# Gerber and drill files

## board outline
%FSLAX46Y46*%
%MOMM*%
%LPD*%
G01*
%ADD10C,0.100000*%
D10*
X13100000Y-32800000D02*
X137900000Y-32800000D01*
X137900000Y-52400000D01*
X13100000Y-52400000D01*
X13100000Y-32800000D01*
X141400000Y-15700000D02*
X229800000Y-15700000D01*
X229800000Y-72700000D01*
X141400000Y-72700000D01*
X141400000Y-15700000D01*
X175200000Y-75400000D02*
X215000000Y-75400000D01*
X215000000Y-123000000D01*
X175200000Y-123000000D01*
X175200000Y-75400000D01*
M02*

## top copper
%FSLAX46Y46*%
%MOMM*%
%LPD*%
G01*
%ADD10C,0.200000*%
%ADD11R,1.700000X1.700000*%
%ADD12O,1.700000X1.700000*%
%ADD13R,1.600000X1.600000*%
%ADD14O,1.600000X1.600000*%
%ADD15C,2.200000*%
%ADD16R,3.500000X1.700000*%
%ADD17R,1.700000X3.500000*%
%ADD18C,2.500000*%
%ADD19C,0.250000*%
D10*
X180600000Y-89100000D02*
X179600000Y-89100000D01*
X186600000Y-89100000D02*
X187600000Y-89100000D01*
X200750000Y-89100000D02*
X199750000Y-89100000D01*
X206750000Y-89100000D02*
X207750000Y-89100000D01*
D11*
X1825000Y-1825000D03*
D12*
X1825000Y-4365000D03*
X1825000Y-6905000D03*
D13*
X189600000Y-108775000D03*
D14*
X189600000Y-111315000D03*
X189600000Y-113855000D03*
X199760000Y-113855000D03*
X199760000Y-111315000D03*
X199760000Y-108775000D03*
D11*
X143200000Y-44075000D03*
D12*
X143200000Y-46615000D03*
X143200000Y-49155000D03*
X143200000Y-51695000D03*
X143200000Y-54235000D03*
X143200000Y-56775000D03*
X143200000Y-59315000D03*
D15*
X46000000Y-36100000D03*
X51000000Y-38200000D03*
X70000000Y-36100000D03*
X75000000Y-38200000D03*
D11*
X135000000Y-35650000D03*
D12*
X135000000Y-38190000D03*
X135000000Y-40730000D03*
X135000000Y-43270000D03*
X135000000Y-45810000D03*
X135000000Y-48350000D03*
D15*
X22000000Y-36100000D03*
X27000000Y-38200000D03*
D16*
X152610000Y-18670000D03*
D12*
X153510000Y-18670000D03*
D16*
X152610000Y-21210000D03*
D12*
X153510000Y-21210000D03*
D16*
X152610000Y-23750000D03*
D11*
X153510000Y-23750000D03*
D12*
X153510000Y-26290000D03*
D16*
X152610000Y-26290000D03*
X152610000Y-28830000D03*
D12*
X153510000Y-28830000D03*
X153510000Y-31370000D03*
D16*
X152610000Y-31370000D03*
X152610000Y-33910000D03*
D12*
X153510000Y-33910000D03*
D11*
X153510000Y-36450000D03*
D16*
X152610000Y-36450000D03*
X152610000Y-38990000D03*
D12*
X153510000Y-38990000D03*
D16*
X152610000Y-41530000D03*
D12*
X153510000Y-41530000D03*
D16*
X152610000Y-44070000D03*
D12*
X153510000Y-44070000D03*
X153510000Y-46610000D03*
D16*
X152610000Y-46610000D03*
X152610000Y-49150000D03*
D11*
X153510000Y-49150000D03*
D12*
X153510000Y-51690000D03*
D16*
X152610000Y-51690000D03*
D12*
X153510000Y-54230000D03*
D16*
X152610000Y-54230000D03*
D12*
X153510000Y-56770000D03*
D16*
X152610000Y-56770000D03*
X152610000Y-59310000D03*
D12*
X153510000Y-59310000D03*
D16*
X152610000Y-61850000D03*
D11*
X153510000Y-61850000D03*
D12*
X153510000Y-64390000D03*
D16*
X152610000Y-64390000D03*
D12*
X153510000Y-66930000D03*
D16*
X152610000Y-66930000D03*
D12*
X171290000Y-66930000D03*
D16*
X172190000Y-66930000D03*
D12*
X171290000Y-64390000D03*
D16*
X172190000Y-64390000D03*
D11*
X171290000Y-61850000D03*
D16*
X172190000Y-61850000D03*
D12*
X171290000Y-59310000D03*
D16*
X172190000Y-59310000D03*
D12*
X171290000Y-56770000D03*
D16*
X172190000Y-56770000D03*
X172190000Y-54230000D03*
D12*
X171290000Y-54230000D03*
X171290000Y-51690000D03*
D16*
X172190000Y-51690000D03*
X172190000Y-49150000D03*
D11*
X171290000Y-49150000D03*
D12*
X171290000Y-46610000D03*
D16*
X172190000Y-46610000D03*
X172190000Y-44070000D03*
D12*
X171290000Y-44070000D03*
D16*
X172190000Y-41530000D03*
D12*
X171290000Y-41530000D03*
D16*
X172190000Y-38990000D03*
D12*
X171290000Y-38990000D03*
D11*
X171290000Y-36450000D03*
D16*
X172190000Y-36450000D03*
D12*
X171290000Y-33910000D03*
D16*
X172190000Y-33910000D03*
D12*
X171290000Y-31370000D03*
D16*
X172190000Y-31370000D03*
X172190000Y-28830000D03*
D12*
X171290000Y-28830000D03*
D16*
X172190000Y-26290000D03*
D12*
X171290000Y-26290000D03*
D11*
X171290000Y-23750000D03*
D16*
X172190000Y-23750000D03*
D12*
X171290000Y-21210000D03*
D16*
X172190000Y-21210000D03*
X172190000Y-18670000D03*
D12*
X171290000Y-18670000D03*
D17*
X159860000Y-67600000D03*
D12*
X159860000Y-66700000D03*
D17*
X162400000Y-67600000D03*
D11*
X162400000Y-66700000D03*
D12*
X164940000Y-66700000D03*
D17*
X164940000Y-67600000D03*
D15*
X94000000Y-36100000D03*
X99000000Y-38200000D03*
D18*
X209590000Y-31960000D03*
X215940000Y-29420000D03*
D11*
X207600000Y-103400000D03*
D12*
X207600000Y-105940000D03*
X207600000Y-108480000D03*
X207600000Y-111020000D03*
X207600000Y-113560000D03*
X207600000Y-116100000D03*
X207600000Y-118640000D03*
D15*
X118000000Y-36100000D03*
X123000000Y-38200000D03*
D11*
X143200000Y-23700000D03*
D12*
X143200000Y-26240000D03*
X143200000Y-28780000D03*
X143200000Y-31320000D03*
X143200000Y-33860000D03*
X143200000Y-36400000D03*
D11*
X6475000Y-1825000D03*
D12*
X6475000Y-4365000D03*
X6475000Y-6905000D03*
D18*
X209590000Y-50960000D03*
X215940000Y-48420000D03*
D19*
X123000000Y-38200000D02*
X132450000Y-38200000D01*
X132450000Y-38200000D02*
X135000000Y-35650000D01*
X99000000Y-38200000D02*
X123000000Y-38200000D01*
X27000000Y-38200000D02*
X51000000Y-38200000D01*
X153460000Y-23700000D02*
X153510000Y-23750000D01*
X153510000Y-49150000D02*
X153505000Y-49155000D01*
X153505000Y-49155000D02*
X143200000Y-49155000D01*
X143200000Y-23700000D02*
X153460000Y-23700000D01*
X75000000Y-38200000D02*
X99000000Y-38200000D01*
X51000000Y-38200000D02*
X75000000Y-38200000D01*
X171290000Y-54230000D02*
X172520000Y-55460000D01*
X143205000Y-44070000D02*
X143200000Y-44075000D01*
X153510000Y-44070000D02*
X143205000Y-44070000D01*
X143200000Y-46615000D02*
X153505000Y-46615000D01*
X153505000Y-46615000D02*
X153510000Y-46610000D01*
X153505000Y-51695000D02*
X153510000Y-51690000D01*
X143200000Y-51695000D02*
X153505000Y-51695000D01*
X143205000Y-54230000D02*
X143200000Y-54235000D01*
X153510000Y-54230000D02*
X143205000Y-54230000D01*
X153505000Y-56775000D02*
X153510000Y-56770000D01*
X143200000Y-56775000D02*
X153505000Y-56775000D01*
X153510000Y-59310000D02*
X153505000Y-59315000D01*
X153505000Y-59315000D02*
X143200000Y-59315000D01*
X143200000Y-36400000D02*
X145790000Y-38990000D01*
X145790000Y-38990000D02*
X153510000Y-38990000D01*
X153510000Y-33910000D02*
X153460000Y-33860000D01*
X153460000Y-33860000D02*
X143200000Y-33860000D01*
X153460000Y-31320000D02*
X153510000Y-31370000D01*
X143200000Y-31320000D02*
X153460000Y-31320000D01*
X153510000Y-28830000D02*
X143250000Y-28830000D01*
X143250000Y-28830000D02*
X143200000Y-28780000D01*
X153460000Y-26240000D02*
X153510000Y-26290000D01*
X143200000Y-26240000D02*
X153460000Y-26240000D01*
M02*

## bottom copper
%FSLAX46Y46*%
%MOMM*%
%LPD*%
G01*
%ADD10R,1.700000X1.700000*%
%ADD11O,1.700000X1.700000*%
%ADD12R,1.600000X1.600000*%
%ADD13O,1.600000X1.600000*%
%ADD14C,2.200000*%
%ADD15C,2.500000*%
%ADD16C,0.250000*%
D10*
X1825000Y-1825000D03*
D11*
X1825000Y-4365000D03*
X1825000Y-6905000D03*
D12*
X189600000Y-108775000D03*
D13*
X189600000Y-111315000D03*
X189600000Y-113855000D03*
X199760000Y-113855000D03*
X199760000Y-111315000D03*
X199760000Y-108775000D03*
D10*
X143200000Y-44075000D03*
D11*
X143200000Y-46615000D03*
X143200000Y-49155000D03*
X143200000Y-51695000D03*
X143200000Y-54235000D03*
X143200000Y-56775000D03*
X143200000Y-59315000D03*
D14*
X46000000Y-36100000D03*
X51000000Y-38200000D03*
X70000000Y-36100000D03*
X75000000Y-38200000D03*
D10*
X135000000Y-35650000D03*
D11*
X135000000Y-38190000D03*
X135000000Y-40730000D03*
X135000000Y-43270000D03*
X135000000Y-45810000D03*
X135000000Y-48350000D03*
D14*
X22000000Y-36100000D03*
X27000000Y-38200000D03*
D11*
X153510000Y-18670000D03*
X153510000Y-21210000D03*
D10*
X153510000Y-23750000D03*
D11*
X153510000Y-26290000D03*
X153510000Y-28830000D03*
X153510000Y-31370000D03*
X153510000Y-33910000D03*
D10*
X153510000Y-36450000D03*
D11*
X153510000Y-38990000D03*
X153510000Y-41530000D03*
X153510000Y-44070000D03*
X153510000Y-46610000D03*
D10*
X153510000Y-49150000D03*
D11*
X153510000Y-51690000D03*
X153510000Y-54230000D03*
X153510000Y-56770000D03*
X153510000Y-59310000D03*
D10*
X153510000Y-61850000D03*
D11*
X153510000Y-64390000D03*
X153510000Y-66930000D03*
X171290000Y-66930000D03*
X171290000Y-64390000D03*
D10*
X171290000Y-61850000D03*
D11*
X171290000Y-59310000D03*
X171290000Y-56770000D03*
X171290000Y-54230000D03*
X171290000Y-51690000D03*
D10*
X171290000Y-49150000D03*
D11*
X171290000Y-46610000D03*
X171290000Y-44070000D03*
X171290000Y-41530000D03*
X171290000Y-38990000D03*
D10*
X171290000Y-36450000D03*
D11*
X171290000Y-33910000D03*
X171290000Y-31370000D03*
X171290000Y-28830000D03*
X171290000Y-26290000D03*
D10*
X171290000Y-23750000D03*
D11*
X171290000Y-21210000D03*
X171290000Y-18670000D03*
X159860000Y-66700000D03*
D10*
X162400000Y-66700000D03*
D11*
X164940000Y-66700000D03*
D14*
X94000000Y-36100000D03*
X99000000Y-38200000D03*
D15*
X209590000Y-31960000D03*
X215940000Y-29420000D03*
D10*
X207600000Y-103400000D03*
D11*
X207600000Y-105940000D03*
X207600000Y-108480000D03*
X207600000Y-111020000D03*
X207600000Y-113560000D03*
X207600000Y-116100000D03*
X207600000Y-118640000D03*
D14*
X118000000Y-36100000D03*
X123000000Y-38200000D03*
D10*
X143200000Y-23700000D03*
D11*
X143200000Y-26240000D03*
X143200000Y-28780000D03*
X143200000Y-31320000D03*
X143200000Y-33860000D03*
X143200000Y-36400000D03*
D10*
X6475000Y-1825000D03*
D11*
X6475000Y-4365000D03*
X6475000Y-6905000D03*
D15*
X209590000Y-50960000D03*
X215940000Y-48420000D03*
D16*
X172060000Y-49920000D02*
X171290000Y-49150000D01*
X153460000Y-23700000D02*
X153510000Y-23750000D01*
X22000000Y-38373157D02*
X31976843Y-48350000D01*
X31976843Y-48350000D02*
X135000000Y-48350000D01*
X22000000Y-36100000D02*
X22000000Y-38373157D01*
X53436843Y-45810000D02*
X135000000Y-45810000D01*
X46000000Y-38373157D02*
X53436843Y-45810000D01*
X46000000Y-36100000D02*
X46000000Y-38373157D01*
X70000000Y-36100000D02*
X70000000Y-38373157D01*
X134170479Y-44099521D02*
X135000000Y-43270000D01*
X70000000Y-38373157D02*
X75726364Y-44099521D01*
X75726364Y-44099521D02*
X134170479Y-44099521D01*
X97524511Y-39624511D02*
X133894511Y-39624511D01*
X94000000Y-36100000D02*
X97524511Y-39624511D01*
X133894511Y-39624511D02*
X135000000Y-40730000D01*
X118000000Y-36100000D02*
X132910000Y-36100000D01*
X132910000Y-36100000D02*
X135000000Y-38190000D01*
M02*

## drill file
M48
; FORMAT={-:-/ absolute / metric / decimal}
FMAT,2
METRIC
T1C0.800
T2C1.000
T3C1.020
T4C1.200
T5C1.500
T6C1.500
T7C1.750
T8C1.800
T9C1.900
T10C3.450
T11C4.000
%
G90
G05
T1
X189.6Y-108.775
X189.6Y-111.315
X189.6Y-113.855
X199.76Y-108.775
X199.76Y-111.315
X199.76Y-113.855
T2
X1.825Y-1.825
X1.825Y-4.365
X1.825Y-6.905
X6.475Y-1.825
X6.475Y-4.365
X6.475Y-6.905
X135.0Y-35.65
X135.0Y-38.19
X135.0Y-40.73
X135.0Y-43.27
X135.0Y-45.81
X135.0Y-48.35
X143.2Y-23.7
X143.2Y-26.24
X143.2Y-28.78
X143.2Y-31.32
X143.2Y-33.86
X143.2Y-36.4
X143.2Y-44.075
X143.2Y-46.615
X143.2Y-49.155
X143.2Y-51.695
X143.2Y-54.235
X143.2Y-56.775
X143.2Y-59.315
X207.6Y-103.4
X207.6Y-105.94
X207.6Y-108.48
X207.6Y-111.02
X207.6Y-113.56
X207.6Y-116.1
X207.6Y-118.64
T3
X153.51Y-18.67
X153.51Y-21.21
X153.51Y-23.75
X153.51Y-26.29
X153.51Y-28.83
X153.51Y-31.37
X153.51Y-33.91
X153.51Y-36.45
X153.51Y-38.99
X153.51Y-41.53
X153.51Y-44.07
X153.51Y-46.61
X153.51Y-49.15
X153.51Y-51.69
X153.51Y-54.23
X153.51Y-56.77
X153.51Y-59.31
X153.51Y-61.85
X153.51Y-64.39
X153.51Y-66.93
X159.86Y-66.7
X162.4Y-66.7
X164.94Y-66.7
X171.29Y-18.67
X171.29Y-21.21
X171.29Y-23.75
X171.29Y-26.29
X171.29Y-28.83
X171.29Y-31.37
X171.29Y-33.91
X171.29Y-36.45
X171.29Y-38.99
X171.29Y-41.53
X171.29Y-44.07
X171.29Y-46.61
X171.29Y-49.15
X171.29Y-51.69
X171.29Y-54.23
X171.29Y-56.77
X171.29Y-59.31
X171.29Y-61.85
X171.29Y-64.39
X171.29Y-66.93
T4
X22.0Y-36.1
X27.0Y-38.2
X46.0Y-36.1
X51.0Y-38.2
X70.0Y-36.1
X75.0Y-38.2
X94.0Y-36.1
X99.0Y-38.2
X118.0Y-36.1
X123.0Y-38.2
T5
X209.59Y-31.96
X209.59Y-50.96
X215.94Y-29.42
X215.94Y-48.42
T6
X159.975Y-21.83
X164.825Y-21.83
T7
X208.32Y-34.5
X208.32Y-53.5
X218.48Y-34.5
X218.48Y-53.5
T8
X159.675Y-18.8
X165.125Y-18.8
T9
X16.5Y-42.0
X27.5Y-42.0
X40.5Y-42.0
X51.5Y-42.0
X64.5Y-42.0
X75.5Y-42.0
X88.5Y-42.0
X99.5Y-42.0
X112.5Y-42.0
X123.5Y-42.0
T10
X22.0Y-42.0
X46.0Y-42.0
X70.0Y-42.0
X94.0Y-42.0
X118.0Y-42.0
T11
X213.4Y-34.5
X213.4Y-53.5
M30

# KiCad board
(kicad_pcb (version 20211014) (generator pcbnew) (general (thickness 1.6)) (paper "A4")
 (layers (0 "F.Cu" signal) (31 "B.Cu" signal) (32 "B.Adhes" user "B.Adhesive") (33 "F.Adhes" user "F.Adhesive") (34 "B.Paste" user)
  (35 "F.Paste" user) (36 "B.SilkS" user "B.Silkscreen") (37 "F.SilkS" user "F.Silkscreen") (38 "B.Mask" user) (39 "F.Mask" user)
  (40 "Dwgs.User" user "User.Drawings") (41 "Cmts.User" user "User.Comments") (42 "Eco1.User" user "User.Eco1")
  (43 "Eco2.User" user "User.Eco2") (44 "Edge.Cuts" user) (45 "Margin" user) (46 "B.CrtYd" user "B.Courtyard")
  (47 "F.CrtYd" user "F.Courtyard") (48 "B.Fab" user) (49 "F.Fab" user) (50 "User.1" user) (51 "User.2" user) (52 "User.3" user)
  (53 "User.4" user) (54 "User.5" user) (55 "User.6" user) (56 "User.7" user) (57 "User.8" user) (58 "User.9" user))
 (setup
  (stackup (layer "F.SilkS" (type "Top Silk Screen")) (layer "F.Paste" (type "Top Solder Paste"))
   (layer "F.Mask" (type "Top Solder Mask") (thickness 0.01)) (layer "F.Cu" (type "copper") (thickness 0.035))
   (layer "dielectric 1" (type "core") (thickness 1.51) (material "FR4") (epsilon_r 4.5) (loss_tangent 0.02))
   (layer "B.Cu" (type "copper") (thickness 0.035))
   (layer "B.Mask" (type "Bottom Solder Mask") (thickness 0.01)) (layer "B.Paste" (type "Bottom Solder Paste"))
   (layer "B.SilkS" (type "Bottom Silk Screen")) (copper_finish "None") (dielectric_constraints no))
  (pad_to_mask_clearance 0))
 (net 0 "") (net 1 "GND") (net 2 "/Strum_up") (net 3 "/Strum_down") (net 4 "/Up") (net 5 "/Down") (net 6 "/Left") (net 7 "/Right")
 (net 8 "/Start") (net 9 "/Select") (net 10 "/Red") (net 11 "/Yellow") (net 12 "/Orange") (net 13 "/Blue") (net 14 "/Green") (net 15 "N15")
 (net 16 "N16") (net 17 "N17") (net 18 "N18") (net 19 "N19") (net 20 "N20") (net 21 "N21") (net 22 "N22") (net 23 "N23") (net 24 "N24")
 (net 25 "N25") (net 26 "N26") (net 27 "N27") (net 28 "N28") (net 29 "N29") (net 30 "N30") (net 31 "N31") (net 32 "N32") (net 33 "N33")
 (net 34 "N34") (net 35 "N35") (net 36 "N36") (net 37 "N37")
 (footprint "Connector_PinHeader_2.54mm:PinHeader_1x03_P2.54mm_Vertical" (layer "F.Cu") (at 1.825 1.825)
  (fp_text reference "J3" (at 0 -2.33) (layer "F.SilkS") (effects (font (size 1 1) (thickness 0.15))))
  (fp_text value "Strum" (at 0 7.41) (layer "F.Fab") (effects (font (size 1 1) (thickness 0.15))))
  (pad "1" thru_hole rect (at 0 0) (size 1.7 1.7) (drill 1) (layers *.Cu *.Mask) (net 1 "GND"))
  (pad "2" thru_hole oval (at 0 2.54) (size 1.7 1.7) (drill 1) (layers *.Cu *.Mask) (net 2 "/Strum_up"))
  (pad "3" thru_hole oval (at 0 5.08) (size 1.7 1.7) (drill 1) (layers *.Cu *.Mask) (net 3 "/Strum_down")))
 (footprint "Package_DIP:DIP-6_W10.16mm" (layer "F.Cu") (at 189.6 108.775)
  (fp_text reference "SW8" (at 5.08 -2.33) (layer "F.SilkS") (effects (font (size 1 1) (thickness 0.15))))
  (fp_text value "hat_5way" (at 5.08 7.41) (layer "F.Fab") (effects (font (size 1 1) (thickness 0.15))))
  (pad "1" thru_hole rect (at 0 0) (size 1.6 1.6) (drill 0.8) (layers *.Cu *.Mask) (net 1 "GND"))
  (pad "2" thru_hole oval (at 0 2.54) (size 1.6 1.6) (drill 0.8) (layers *.Cu *.Mask) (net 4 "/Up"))
  (pad "3" thru_hole oval (at 0 5.08) (size 1.6 1.6) (drill 0.8) (layers *.Cu *.Mask) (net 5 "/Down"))
  (pad "4" thru_hole oval (at 10.16 5.08) (size 1.6 1.6) (drill 0.8) (layers *.Cu *.Mask) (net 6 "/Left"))
  (pad "5" thru_hole oval (at 10.16 2.54) (size 1.6 1.6) (drill 0.8) (layers *.Cu *.Mask) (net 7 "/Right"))
  (pad "6" thru_hole oval (at 10.16 0) (size 1.6 1.6) (drill 0.8) (layers *.Cu *.Mask)))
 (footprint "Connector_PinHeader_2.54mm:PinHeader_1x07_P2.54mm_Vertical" (layer "F.Cu") (at 143.2 44.075)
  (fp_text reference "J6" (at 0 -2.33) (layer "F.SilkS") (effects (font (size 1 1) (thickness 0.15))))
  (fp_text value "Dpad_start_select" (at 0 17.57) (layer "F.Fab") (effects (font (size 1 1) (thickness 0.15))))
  (pad "1" thru_hole rect (at 0 0) (size 1.7 1.7) (drill 1) (layers *.Cu *.Mask) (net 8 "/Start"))
  (pad "2" thru_hole oval (at 0 2.54) (size 1.7 1.7) (drill 1) (layers *.Cu *.Mask) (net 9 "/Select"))
  (pad "3" thru_hole oval (at 0 5.08) (size 1.7 1.7) (drill 1) (layers *.Cu *.Mask) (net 1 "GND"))
  (pad "4" thru_hole oval (at 0 7.62) (size 1.7 1.7) (drill 1) (layers *.Cu *.Mask) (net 4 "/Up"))
  (pad "5" thru_hole oval (at 0 10.16) (size 1.7 1.7) (drill 1) (layers *.Cu *.Mask) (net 5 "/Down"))
  (pad "6" thru_hole oval (at 0 12.7) (size 1.7 1.7) (drill 1) (layers *.Cu *.Mask) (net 6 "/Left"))
  (pad "7" thru_hole oval (at 0 15.24) (size 1.7 1.7) (drill 1) (layers *.Cu *.Mask) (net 7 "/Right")))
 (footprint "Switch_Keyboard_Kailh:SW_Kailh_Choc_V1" (layer "F.Cu") (at 46 42)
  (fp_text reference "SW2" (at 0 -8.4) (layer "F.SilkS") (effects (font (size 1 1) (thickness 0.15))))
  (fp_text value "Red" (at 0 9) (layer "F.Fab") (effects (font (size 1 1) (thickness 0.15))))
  (pad "" np_thru_hole circle locked (at 5.5 0) (size 1.9 1.9) (drill 1.9) (layers *.Cu *.Mask))
  (pad "" np_thru_hole circle locked (at -5.5 0) (size 1.9 1.9) (drill 1.9) (layers *.Cu *.Mask))
  (pad "" smd circle locked (at 0 -5.9) (size 1.25 1.25) (layers "F.Mask"))
  (pad "" np_thru_hole circle locked (at 0 0) (size 3.45 3.45) (drill 3.45) (layers *.Cu *.Mask))
  (pad "" smd circle locked (at 5 -3.8) (size 1.25 1.25) (layers "F.Mask"))
  (pad "1" thru_hole circle locked (at 0 -5.9) (size 2.2 2.2) (drill 1.2) (layers *.Cu "B.Mask") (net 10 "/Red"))
  (pad "2" thru_hole circle locked (at 5 -3.8) (size 2.2 2.2) (drill 1.2) (layers *.Cu "B.Mask") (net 1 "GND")))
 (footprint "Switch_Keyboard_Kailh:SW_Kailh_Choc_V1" (layer "F.Cu") (at 70 42)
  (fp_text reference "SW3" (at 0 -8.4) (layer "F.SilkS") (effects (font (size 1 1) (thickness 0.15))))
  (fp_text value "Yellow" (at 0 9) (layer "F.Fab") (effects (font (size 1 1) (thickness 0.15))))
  (pad "" np_thru_hole circle locked (at -5.5 0) (size 1.9 1.9) (drill 1.9) (layers *.Cu *.Mask))
  (pad "" np_thru_hole circle locked (at 0 0) (size 3.45 3.45) (drill 3.45) (layers *.Cu *.Mask))
  (pad "" smd circle locked (at 0 -5.9) (size 1.25 1.25) (layers "F.Mask"))
  (pad "" smd circle locked (at 5 -3.8) (size 1.25 1.25) (layers "F.Mask"))
  (pad "" np_thru_hole circle locked (at 5.5 0) (size 1.9 1.9) (drill 1.9) (layers *.Cu *.Mask))
  (pad "1" thru_hole circle locked (at 0 -5.9) (size 2.2 2.2) (drill 1.2) (layers *.Cu "B.Mask") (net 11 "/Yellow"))
  (pad "2" thru_hole circle locked (at 5 -3.8) (size 2.2 2.2) (drill 1.2) (layers *.Cu "B.Mask") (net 1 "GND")))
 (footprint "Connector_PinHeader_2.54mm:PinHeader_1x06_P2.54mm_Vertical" (layer "F.Cu") (at 135 35.65)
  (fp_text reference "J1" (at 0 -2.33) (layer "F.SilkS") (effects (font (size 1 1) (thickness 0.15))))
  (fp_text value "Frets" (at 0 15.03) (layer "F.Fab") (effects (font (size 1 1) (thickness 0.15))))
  (pad "1" thru_hole rect (at 0 0) (size 1.7 1.7) (drill 1) (layers *.Cu *.Mask) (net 1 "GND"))
  (pad "2" thru_hole oval (at 0 2.54) (size 1.7 1.7) (drill 1) (layers *.Cu *.Mask) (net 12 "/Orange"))
  (pad "3" thru_hole oval (at 0 5.08) (size 1.7 1.7) (drill 1) (layers *.Cu *.Mask) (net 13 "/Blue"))
  (pad "4" thru_hole oval (at 0 7.62) (size 1.7 1.7) (drill 1) (layers *.Cu *.Mask) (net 11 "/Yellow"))
  (pad "5" thru_hole oval (at 0 10.16) (size 1.7 1.7) (drill 1) (layers *.Cu *.Mask) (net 10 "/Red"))
  (pad "6" thru_hole oval (at 0 12.7) (size 1.7 1.7) (drill 1) (layers *.Cu *.Mask) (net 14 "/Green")))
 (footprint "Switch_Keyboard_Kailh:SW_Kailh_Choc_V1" (layer "F.Cu") (at 22 42)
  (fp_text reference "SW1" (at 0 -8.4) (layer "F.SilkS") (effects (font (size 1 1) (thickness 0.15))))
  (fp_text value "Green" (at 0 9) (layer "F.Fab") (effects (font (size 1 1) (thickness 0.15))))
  (pad "" smd circle locked (at 0 -5.9) (size 1.25 1.25) (layers "F.Mask"))
  (pad "" smd circle locked (at 5 -3.8) (size 1.25 1.25) (layers "F.Mask"))
  (pad "" np_thru_hole circle locked (at 0 0) (size 3.45 3.45) (drill 3.45) (layers *.Cu *.Mask))
  (pad "" np_thru_hole circle locked (at 5.5 0) (size 1.9 1.9) (drill 1.9) (layers *.Cu *.Mask))
  (pad "" np_thru_hole circle locked (at -5.5 0) (size 1.9 1.9) (drill 1.9) (layers *.Cu *.Mask))
  (pad "1" thru_hole circle locked (at 0 -5.9) (size 2.2 2.2) (drill 1.2) (layers *.Cu "B.Mask") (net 14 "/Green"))
  (pad "2" thru_hole circle locked (at 5 -3.8) (size 2.2 2.2) (drill 1.2) (layers *.Cu "B.Mask") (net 1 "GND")))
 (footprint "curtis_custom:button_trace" (layer "F.Cu") (at 183.6 89.1)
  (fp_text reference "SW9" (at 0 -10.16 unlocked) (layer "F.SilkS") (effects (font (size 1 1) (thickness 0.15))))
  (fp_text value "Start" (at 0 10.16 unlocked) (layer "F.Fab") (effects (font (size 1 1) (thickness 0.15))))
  (fp_line (start -3 0) (end -4 0) (layer "F.Cu") (width 0.2)) (fp_line (start 3 0) (end 4 0) (layer "F.Cu") (width 0.2)))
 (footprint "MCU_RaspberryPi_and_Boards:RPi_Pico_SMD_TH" (layer "F.Cu") (at 162.4 42.8)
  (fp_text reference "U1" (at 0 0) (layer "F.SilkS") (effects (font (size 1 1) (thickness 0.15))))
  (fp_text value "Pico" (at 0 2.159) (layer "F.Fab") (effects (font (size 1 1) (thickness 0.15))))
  (pad "" np_thru_hole oval (at -2.725 -24) (size 1.8 1.8) (drill 1.8) (layers *.Cu *.Mask))
  (pad "" np_thru_hole oval (at 2.425 -20.97) (size 1.5 1.5) (drill 1.5) (layers *.Cu *.Mask))
  (pad "" np_thru_hole oval (at -2.425 -20.97) (size 1.5 1.5) (drill 1.5) (layers *.Cu *.Mask))
  (pad "" np_thru_hole oval (at 2.725 -24) (size 1.8 1.8) (drill 1.8) (layers *.Cu *.Mask))
  (pad "1" smd rect (at -8.89 -24.13) (size 3.5 1.7) (drill (offset -0.9 0)) (layers "F.Cu" "F.Mask") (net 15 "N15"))
  (pad "1" thru_hole oval (at -8.89 -24.13) (size 1.7 1.7) (drill 1.02) (layers *.Cu *.Mask) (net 15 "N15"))
  (pad "2" smd rect (at -8.89 -21.59) (size 3.5 1.7) (drill (offset -0.9 0)) (layers "F.Cu" "F.Mask") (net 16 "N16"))
  (pad "2" thru_hole oval (at -8.89 -21.59) (size 1.7 1.7) (drill 1.02) (layers *.Cu *.Mask) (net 16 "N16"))
  (pad "3" smd rect (at -8.89 -19.05) (size 3.5 1.7) (drill (offset -0.9 0)) (layers "F.Cu" "F.Mask") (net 1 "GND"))
  (pad "3" thru_hole rect (at -8.89 -19.05) (size 1.7 1.7) (drill 1.02) (layers *.Cu *.Mask) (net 1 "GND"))
  (pad "4" thru_hole oval (at -8.89 -16.51) (size 1.7 1.7) (drill 1.02) (layers *.Cu *.Mask) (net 12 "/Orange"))
  (pad "4" smd rect (at -8.89 -16.51) (size 3.5 1.7) (drill (offset -0.9 0)) (layers "F.Cu" "F.Mask") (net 12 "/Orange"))
  (pad "5" smd rect (at -8.89 -13.97) (size 3.5 1.7) (drill (offset -0.9 0)) (layers "F.Cu" "F.Mask") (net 13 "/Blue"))
  (pad "5" thru_hole oval (at -8.89 -13.97) (size 1.7 1.7) (drill 1.02) (layers *.Cu *.Mask) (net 13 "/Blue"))
  (pad "6" thru_hole oval (at -8.89 -11.43) (size 1.7 1.7) (drill 1.02) (layers *.Cu *.Mask) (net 11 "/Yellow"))
  (pad "6" smd rect (at -8.89 -11.43) (size 3.5 1.7) (drill (offset -0.9 0)) (layers "F.Cu" "F.Mask") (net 11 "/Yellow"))
  (pad "7" smd rect (at -8.89 -8.89) (size 3.5 1.7) (drill (offset -0.9 0)) (layers "F.Cu" "F.Mask") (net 10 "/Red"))
  (pad "7" thru_hole oval (at -8.89 -8.89) (size 1.7 1.7) (drill 1.02) (layers *.Cu *.Mask) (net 10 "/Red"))
  (pad "8" thru_hole rect (at -8.89 -6.35) (size 1.7 1.7) (drill 1.02) (layers *.Cu *.Mask) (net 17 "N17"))
  (pad "8" smd rect (at -8.89 -6.35) (size 3.5 1.7) (drill (offset -0.9 0)) (layers "F.Cu" "F.Mask") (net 17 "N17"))
  (pad "9" smd rect (at -8.89 -3.81) (size 3.5 1.7) (drill (offset -0.9 0)) (layers "F.Cu" "F.Mask") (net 14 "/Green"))
  (pad "9" thru_hole oval (at -8.89 -3.81) (size 1.7 1.7) (drill 1.02) (layers *.Cu *.Mask) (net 14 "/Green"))
  (pad "10" smd rect (at -8.89 -1.27) (size 3.5 1.7) (drill (offset -0.9 0)) (layers "F.Cu" "F.Mask") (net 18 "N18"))
  (pad "10" thru_hole oval (at -8.89 -1.27) (size 1.7 1.7) (drill 1.02) (layers *.Cu *.Mask) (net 18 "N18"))
  (pad "11" smd rect (at -8.89 1.27) (size 3.5 1.7) (drill (offset -0.9 0)) (layers "F.Cu" "F.Mask") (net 8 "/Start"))
  (pad "11" thru_hole oval (at -8.89 1.27) (size 1.7 1.7) (drill 1.02) (layers *.Cu *.Mask) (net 8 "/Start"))
  (pad "12" thru_hole oval (at -8.89 3.81) (size 1.7 1.7) (drill 1.02) (layers *.Cu *.Mask) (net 9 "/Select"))
  (pad "12" smd rect (at -8.89 3.81) (size 3.5 1.7) (drill (offset -0.9 0)) (layers "F.Cu" "F.Mask") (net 9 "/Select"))
  (pad "13" smd rect (at -8.89 6.35) (size 3.5 1.7) (drill (offset -0.9 0)) (layers "F.Cu" "F.Mask") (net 1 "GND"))
  (pad "13" thru_hole rect (at -8.89 6.35) (size 1.7 1.7) (drill 1.02) (layers *.Cu *.Mask) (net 1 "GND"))
  (pad "14" thru_hole oval (at -8.89 8.89) (size 1.7 1.7) (drill 1.02) (layers *.Cu *.Mask) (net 4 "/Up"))
  (pad "14" smd rect (at -8.89 8.89) (size 3.5 1.7) (drill (offset -0.9 0)) (layers "F.Cu" "F.Mask") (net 4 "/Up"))
  (pad "15" thru_hole oval (at -8.89 11.43) (size 1.7 1.7) (drill 1.02) (layers *.Cu *.Mask) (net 5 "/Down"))
  (pad "15" smd rect (at -8.89 11.43) (size 3.5 1.7) (drill (offset -0.9 0)) (layers "F.Cu" "F.Mask") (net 5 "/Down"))
  (pad "16" thru_hole oval (at -8.89 13.97) (size 1.7 1.7) (drill 1.02) (layers *.Cu *.Mask) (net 6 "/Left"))
  (pad "16" smd rect (at -8.89 13.97) (size 3.5 1.7) (drill (offset -0.9 0)) (layers "F.Cu" "F.Mask") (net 6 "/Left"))
  (pad "17" smd rect (at -8.89 16.51) (size 3.5 1.7) (drill (offset -0.9 0)) (layers "F.Cu" "F.Mask") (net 7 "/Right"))
  (pad "17" thru_hole oval (at -8.89 16.51) (size 1.7 1.7) (drill 1.02) (layers *.Cu *.Mask) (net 7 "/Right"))
  (pad "18" smd rect (at -8.89 19.05) (size 3.5 1.7) (drill (offset -0.9 0)) (layers "F.Cu" "F.Mask") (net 1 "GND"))
  (pad "18" thru_hole rect (at -8.89 19.05) (size 1.7 1.7) (drill 1.02) (layers *.Cu *.Mask) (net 1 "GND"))
  (pad "19" thru_hole oval (at -8.89 21.59) (size 1.7 1.7) (drill 1.02) (layers *.Cu *.Mask) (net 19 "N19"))
  (pad "19" smd rect (at -8.89 21.59) (size 3.5 1.7) (drill (offset -0.9 0)) (layers "F.Cu" "F.Mask") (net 19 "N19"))
  (pad "20" thru_hole oval (at -8.89 24.13) (size 1.7 1.7) (drill 1.02) (layers *.Cu *.Mask) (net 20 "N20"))
  (pad "20" smd rect (at -8.89 24.13) (size 3.5 1.7) (drill (offset -0.9 0)) (layers "F.Cu" "F.Mask") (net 20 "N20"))
  (pad "21" thru_hole oval (at 8.89 24.13) (size 1.7 1.7) (drill 1.02) (layers *.Cu *.Mask) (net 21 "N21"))
  (pad "21" smd rect (at 8.89 24.13) (size 3.5 1.7) (drill (offset 0.9 0)) (layers "F.Cu" "F.Mask") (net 21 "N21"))
  (pad "22" thru_hole oval (at 8.89 21.59) (size 1.7 1.7) (drill 1.02) (layers *.Cu *.Mask) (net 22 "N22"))
  (pad "22" smd rect (at 8.89 21.59) (size 3.5 1.7) (drill (offset 0.9 0)) (layers "F.Cu" "F.Mask") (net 22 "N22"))
  (pad "23" thru_hole rect (at 8.89 19.05) (size 1.7 1.7) (drill 1.02) (layers *.Cu *.Mask) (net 1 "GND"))
  (pad "23" smd rect (at 8.89 19.05) (size 3.5 1.7) (drill (offset 0.9 0)) (layers "F.Cu" "F.Mask") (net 1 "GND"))
  (pad "24" thru_hole oval (at 8.89 16.51) (size 1.7 1.7) (drill 1.02) (layers *.Cu *.Mask) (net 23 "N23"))
  (pad "24" smd rect (at 8.89 16.51) (size 3.5 1.7) (drill (offset 0.9 0)) (layers "F.Cu" "F.Mask") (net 23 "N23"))
  (pad "25" thru_hole oval (at 8.89 13.97) (size 1.7 1.7) (drill 1.02) (layers *.Cu *.Mask) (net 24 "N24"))
  (pad "25" smd rect (at 8.89 13.97) (size 3.5 1.7) (drill (offset 0.9 0)) (layers "F.Cu" "F.Mask") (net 24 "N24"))
  (pad "26" smd rect (at 8.89 11.43) (size 3.5 1.7) (drill (offset 0.9 0)) (layers "F.Cu" "F.Mask") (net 3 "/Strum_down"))
  (pad "26" thru_hole oval (at 8.89 11.43) (size 1.7 1.7) (drill 1.02) (layers *.Cu *.Mask) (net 3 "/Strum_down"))
  (pad "27" thru_hole oval (at 8.89 8.89) (size 1.7 1.7) (drill 1.02) (layers *.Cu *.Mask) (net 2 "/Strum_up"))
  (pad "27" smd rect (at 8.89 8.89) (size 3.5 1.7) (drill (offset 0.9 0)) (layers "F.Cu" "F.Mask") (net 2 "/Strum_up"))
  (pad "28" smd rect (at 8.89 6.35) (size 3.5 1.7) (drill (offset 0.9 0)) (layers "F.Cu" "F.Mask") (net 1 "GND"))
  (pad "28" thru_hole rect (at 8.89 6.35) (size 1.7 1.7) (drill 1.02) (layers *.Cu *.Mask) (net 1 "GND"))
  (pad "29" thru_hole oval (at 8.89 3.81) (size 1.7 1.7) (drill 1.02) (layers *.Cu *.Mask) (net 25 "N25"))
  (pad "29" smd rect (at 8.89 3.81) (size 3.5 1.7) (drill (offset 0.9 0)) (layers "F.Cu" "F.Mask") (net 25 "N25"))
  (pad "30" smd rect (at 8.89 1.27) (size 3.5 1.7) (drill (offset 0.9 0)) (layers "F.Cu" "F.Mask") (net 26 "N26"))
  (pad "30" thru_hole oval (at 8.89 1.27) (size 1.7 1.7) (drill 1.02) (layers *.Cu *.Mask) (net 26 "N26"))
  (pad "31" smd rect (at 8.89 -1.27) (size 3.5 1.7) (drill (offset 0.9 0)) (layers "F.Cu" "F.Mask") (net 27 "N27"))
  (pad "31" thru_hole oval (at 8.89 -1.27) (size 1.7 1.7) (drill 1.02) (layers *.Cu *.Mask) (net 27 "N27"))
  (pad "32" smd rect (at 8.89 -3.81) (size 3.5 1.7) (drill (offset 0.9 0)) (layers "F.Cu" "F.Mask") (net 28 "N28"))
  (pad "32" thru_hole oval (at 8.89 -3.81) (size 1.7 1.7) (drill 1.02) (layers *.Cu *.Mask) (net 28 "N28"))
  (pad "33" thru_hole rect (at 8.89 -6.35) (size 1.7 1.7) (drill 1.02) (layers *.Cu *.Mask) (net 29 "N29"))
  (pad "33" smd rect (at 8.89 -6.35) (size 3.5 1.7) (drill (offset 0.9 0)) (layers "F.Cu" "F.Mask") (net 29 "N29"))
  (pad "34" thru_hole oval (at 8.89 -8.89) (size 1.7 1.7) (drill 1.02) (layers *.Cu *.Mask) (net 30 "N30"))
  (pad "34" smd rect (at 8.89 -8.89) (size 3.5 1.7) (drill (offset 0.9 0)) (layers "F.Cu" "F.Mask") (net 30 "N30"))
  (pad "35" thru_hole oval (at 8.89 -11.43) (size 1.7 1.7) (drill 1.02) (layers *.Cu *.Mask) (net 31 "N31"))
  (pad "35" smd rect (at 8.89 -11.43) (size 3.5 1.7) (drill (offset 0.9 0)) (layers "F.Cu" "F.Mask") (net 31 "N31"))
  (pad "36" smd rect (at 8.89 -13.97) (size 3.5 1.7) (drill (offset 0.9 0)) (layers "F.Cu" "F.Mask") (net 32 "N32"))
  (pad "36" thru_hole oval (at 8.89 -13.97) (size 1.7 1.7) (drill 1.02) (layers *.Cu *.Mask) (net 32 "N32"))
  (pad "37" smd rect (at 8.89 -16.51) (size 3.5 1.7) (drill (offset 0.9 0)) (layers "F.Cu" "F.Mask") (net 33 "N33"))
  (pad "37" thru_hole oval (at 8.89 -16.51) (size 1.7 1.7) (drill 1.02) (layers *.Cu *.Mask) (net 33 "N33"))
  (pad "38" thru_hole rect (at 8.89 -19.05) (size 1.7 1.7) (drill 1.02) (layers *.Cu *.Mask) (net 1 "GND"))
  (pad "38" smd rect (at 8.89 -19.05) (size 3.5 1.7) (drill (offset 0.9 0)) (layers "F.Cu" "F.Mask") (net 1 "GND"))
  (pad "39" thru_hole oval (at 8.89 -21.59) (size 1.7 1.7) (drill 1.02) (layers *.Cu *.Mask) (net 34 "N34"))
  (pad "39" smd rect (at 8.89 -21.59) (size 3.5 1.7) (drill (offset 0.9 0)) (layers "F.Cu" "F.Mask") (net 34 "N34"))
  (pad "40" smd rect (at 8.89 -24.13) (size 3.5 1.7) (drill (offset 0.9 0)) (layers "F.Cu" "F.Mask") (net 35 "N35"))
  (pad "40" thru_hole oval (at 8.89 -24.13) (size 1.7 1.7) (drill 1.02) (layers *.Cu *.Mask) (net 35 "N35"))
  (pad "41" smd rect (at -2.54 23.9 90) (size 3.5 1.7) (drill (offset -0.9 0)) (layers "F.Cu" "F.Mask") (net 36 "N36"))
  (pad "41" thru_hole oval (at -2.54 23.9) (size 1.7 1.7) (drill 1.02) (layers *.Cu *.Mask) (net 36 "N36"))
  (pad "42" smd rect (at 0 23.9 90) (size 3.5 1.7) (drill (offset -0.9 0)) (layers "F.Cu" "F.Mask") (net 1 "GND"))
  (pad "42" thru_hole rect (at 0 23.9) (size 1.7 1.7) (drill 1.02) (layers *.Cu *.Mask) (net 1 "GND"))
  (pad "43" thru_hole oval (at 2.54 23.9) (size 1.7 1.7) (drill 1.02) (layers *.Cu *.Mask) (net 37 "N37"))
  (pad "43" smd rect (at 2.54 23.9 90) (size 3.5 1.7) (drill (offset -0.9 0)) (layers "F.Cu" "F.Mask") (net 37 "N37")))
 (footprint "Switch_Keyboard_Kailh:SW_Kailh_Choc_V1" (layer "F.Cu") (at 94 42)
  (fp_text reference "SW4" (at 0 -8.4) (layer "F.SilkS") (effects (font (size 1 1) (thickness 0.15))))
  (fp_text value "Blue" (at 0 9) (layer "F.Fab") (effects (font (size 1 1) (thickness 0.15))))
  (pad "" np_thru_hole circle locked (at 0 0) (size 3.45 3.45) (drill 3.45) (layers *.Cu *.Mask))
  (pad "" smd circle locked (at 5 -3.8) (size 1.25 1.25) (layers "F.Mask"))
  (pad "" np_thru_hole circle locked (at 5.5 0) (size 1.9 1.9) (drill 1.9) (layers *.Cu *.Mask))
  (pad "" np_thru_hole circle locked (at -5.5 0) (size 1.9 1.9) (drill 1.9) (layers *.Cu *.Mask))
  (pad "" smd circle locked (at 0 -5.9) (size 1.25 1.25) (layers "F.Mask"))
  (pad "1" thru_hole circle locked (at 0 -5.9) (size 2.2 2.2) (drill 1.2) (layers *.Cu "B.Mask") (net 13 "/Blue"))
  (pad "2" thru_hole circle locked (at 5 -3.8) (size 2.2 2.2) (drill 1.2) (layers *.Cu "B.Mask") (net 1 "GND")))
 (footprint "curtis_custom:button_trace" (layer "F.Cu") (at 203.75 89.1)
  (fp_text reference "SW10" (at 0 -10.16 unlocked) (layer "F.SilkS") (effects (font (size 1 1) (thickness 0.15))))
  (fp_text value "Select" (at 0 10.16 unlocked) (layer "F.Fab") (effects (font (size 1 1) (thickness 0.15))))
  (fp_line (start -3 0) (end -4 0) (layer "F.Cu") (width 0.2)) (fp_line (start 3 0) (end 4 0) (layer "F.Cu") (width 0.2)))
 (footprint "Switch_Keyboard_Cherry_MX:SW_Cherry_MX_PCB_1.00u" (layer "F.Cu") (at 213.4 34.5)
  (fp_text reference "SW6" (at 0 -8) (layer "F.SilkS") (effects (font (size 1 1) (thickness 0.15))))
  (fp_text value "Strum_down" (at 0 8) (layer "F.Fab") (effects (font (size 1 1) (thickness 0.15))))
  (pad "" smd circle locked (at 2.54 -5.08) (size 1.55 1.55) (layers "F.Mask"))
  (pad "" np_thru_hole circle locked (at -5.08 0) (size 1.75 1.75) (drill 1.75) (layers *.Cu *.Mask))
  (pad "" np_thru_hole circle locked (at 0 0) (size 4 4) (drill 4) (layers *.Cu *.Mask))
  (pad "" smd circle locked (at -3.81 -2.54) (size 1.55 1.55) (layers "F.Mask"))
  (pad "" np_thru_hole circle locked (at 5.08 0) (size 1.75 1.75) (drill 1.75) (layers *.Cu *.Mask))
  (pad "1" thru_hole circle locked (at -3.81 -2.54) (size 2.5 2.5) (drill 1.5) (layers *.Cu "B.Mask") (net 3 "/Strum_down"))
  (pad "2" thru_hole circle locked (at 2.54 -5.08) (size 2.5 2.5) (drill 1.5) (layers *.Cu "B.Mask") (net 1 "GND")))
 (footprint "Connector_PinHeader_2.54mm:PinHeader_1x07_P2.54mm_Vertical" (layer "F.Cu") (at 207.6 103.4)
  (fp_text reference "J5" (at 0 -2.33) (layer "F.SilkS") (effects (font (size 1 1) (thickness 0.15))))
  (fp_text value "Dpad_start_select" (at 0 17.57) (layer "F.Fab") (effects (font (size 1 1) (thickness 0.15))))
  (pad "1" thru_hole rect (at 0 0) (size 1.7 1.7) (drill 1) (layers *.Cu *.Mask) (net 8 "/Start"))
  (pad "2" thru_hole oval (at 0 2.54) (size 1.7 1.7) (drill 1) (layers *.Cu *.Mask) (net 9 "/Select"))
  (pad "3" thru_hole oval (at 0 5.08) (size 1.7 1.7) (drill 1) (layers *.Cu *.Mask) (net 1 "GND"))
  (pad "4" thru_hole oval (at 0 7.62) (size 1.7 1.7) (drill 1) (layers *.Cu *.Mask) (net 4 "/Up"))
  (pad "5" thru_hole oval (at 0 10.16) (size 1.7 1.7) (drill 1) (layers *.Cu *.Mask) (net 5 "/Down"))
  (pad "6" thru_hole oval (at 0 12.7) (size 1.7 1.7) (drill 1) (layers *.Cu *.Mask) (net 6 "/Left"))
  (pad "7" thru_hole oval (at 0 15.24) (size 1.7 1.7) (drill 1) (layers *.Cu *.Mask) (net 7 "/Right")))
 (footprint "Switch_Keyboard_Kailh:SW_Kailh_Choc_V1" (layer "F.Cu") (at 118 42)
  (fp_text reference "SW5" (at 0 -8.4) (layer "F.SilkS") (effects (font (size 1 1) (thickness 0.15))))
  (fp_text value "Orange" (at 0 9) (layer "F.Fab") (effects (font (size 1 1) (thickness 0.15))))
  (pad "" np_thru_hole circle locked (at 5.5 0) (size 1.9 1.9) (drill 1.9) (layers *.Cu *.Mask))
  (pad "" smd circle locked (at 5 -3.8) (size 1.25 1.25) (layers "F.Mask"))
  (pad "" np_thru_hole circle locked (at 0 0) (size 3.45 3.45) (drill 3.45) (layers *.Cu *.Mask))
  (pad "" smd circle locked (at 0 -5.9) (size 1.25 1.25) (layers "F.Mask"))
  (pad "" np_thru_hole circle locked (at -5.5 0) (size 1.9 1.9) (drill 1.9) (layers *.Cu *.Mask))
  (pad "1" thru_hole circle locked (at 0 -5.9) (size 2.2 2.2) (drill 1.2) (layers *.Cu "B.Mask") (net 12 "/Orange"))
  (pad "2" thru_hole circle locked (at 5 -3.8) (size 2.2 2.2) (drill 1.2) (layers *.Cu "B.Mask") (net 1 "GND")))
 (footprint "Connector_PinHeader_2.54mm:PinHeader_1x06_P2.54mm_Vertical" (layer "F.Cu") (at 143.2 23.7)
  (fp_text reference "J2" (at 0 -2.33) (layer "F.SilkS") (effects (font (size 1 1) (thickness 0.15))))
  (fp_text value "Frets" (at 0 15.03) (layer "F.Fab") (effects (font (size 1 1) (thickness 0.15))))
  (pad "1" thru_hole rect (at 0 0) (size 1.7 1.7) (drill 1) (layers *.Cu *.Mask) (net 1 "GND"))
  (pad "2" thru_hole oval (at 0 2.54) (size 1.7 1.7) (drill 1) (layers *.Cu *.Mask) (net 12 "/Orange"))
  (pad "3" thru_hole oval (at 0 5.08) (size 1.7 1.7) (drill 1) (layers *.Cu *.Mask) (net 13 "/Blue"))
  (pad "4" thru_hole oval (at 0 7.62) (size 1.7 1.7) (drill 1) (layers *.Cu *.Mask) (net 11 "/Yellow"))
  (pad "5" thru_hole oval (at 0 10.16) (size 1.7 1.7) (drill 1) (layers *.Cu *.Mask) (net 10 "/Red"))
  (pad "6" thru_hole oval (at 0 12.7) (size 1.7 1.7) (drill 1) (layers *.Cu *.Mask) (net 14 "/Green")))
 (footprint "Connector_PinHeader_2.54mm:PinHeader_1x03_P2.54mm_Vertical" (layer "F.Cu") (at 6.475 1.825)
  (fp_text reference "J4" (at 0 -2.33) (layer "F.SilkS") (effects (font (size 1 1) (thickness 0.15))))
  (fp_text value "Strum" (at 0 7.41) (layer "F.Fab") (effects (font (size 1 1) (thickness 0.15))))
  (pad "1" thru_hole rect (at 0 0) (size 1.7 1.7) (drill 1) (layers *.Cu *.Mask) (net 1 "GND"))
  (pad "2" thru_hole oval (at 0 2.54) (size 1.7 1.7) (drill 1) (layers *.Cu *.Mask) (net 2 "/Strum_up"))
  (pad "3" thru_hole oval (at 0 5.08) (size 1.7 1.7) (drill 1) (layers *.Cu *.Mask) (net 3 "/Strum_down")))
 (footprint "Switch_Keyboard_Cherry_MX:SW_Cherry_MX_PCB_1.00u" (layer "F.Cu") (at 213.4 53.5)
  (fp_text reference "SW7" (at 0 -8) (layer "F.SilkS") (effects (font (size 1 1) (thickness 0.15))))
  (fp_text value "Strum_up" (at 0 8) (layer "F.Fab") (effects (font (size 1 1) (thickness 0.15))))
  (pad "" np_thru_hole circle locked (at 0 0) (size 4 4) (drill 4) (layers *.Cu *.Mask))
  (pad "" np_thru_hole circle locked (at -5.08 0) (size 1.75 1.75) (drill 1.75) (layers *.Cu *.Mask))
  (pad "" smd circle locked (at -3.81 -2.54) (size 1.55 1.55) (layers "F.Mask"))
  (pad "" smd circle locked (at 2.54 -5.08) (size 1.55 1.55) (layers "F.Mask"))
  (pad "" np_thru_hole circle locked (at 5.08 0) (size 1.75 1.75) (drill 1.75) (layers *.Cu *.Mask))
  (pad "1" thru_hole circle locked (at -3.81 -2.54) (size 2.5 2.5) (drill 1.5) (layers *.Cu "B.Mask") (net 2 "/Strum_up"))
  (pad "2" thru_hole circle locked (at 2.54 -5.08) (size 2.5 2.5) (drill 1.5) (layers *.Cu "B.Mask") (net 1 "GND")))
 (gr_rect (start 13.1 32.8) (end 137.9 52.4) (layer "Edge.Cuts") (width 0.1) (fill none))
 (gr_rect (start 229.8 72.7) (end 141.4 15.7) (layer "Edge.Cuts") (width 0.1) (fill none))
 (gr_rect (start 175.2 75.4) (end 215 123) (layer "Edge.Cuts") (width 0.1) (fill none))
 (segment (start 123 38.2) (end 132.45 38.2) (width 0.25) (layer "F.Cu") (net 1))
 (segment (start 132.45 38.2) (end 135 35.65) (width 0.25) (layer "F.Cu") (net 1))
 (segment (start 99 38.2) (end 123 38.2) (width 0.25) (layer "F.Cu") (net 1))
 (segment (start 27 38.2) (end 51 38.2) (width 0.25) (layer "F.Cu") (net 1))
 (segment (start 153.46 23.7) (end 153.51 23.75) (width 0.25) (layer "F.Cu") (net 1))
 (segment (start 153.51 49.15) (end 153.505 49.155) (width 0.25) (layer "F.Cu") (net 1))
 (segment (start 153.505 49.155) (end 143.2 49.155) (width 0.25) (layer "F.Cu") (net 1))
 (segment (start 143.2 23.7) (end 153.46 23.7) (width 0.25) (layer "F.Cu") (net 1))
 (segment (start 75 38.2) (end 99 38.2) (width 0.25) (layer "F.Cu") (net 1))
 (segment (start 51 38.2) (end 75 38.2) (width 0.25) (layer "F.Cu") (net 1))
 (segment (start 172.06 49.92) (end 171.29 49.15) (width 0.25) (layer "B.Cu") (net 1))
 (segment (start 153.46 23.7) (end 153.51 23.75) (width 0.25) (layer "B.Cu") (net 1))
 (segment (start 171.29 54.23) (end 172.52 55.46) (width 0.25) (layer "F.Cu") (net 3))
 (segment (start 143.205 44.07) (end 143.2 44.075) (width 0.25) (layer "F.Cu") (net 8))
 (segment (start 153.51 44.07) (end 143.205 44.07) (width 0.25) (layer "F.Cu") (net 8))
 (segment (start 143.2 46.615) (end 153.505 46.615) (width 0.25) (layer "F.Cu") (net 9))
 (segment (start 153.505 46.615) (end 153.51 46.61) (width 0.25) (layer "F.Cu") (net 9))
 (segment (start 153.505 51.695) (end 153.51 51.69) (width 0.25) (layer "F.Cu") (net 4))
 (segment (start 143.2 51.695) (end 153.505 51.695) (width 0.25) (layer "F.Cu") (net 4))
 (segment (start 143.205 54.23) (end 143.2 54.235) (width 0.25) (layer "F.Cu") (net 5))
 (segment (start 153.51 54.23) (end 143.205 54.23) (width 0.25) (layer "F.Cu") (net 5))
 (segment (start 153.505 56.775) (end 153.51 56.77) (width 0.25) (layer "F.Cu") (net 6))
 (segment (start 143.2 56.775) (end 153.505 56.775) (width 0.25) (layer "F.Cu") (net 6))
 (segment (start 153.51 59.31) (end 153.505 59.315) (width 0.25) (layer "F.Cu") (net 7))
 (segment (start 153.505 59.315) (end 143.2 59.315) (width 0.25) (layer "F.Cu") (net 7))
 (segment (start 143.2 36.4) (end 145.79 38.99) (width 0.25) (layer "F.Cu") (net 14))
 (segment (start 145.79 38.99) (end 153.51 38.99) (width 0.25) (layer "F.Cu") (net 14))
 (segment (start 22 38.373157) (end 31.976843 48.35) (width 0.25) (layer "B.Cu") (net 14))
 (segment (start 31.976843 48.35) (end 135 48.35) (width 0.25) (layer "B.Cu") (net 14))
 (segment (start 22 36.1) (end 22 38.373157) (width 0.25) (layer "B.Cu") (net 14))
 (segment (start 153.51 33.91) (end 153.46 33.86) (width 0.25) (layer "F.Cu") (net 10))
 (segment (start 153.46 33.86) (end 143.2 33.86) (width 0.25) (layer "F.Cu") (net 10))
 (segment (start 53.436843 45.81) (end 135 45.81) (width 0.25) (layer "B.Cu") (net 10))
 (segment (start 46 38.373157) (end 53.436843 45.81) (width 0.25) (layer "B.Cu") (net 10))
 (segment (start 46 36.1) (end 46 38.373157) (width 0.25) (layer "B.Cu") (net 10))
 (segment (start 153.46 31.32) (end 153.51 31.37) (width 0.25) (layer "F.Cu") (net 11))
 (segment (start 143.2 31.32) (end 153.46 31.32) (width 0.25) (layer "F.Cu") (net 11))
 (segment (start 70 36.1) (end 70 38.373157) (width 0.25) (layer "B.Cu") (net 11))
 (segment (start 134.170479 44.099521) (end 135 43.27) (width 0.25) (layer "B.Cu") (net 11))
 (segment (start 70 38.373157) (end 75.726364 44.099521) (width 0.25) (layer "B.Cu") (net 11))
 (segment (start 75.726364 44.099521) (end 134.170479 44.099521) (width 0.25) (layer "B.Cu") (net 11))
 (segment (start 153.51 28.83) (end 143.25 28.83) (width 0.25) (layer "F.Cu") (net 13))
 (segment (start 143.25 28.83) (end 143.2 28.78) (width 0.25) (layer "F.Cu") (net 13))
 (segment (start 97.524511 39.624511) (end 133.894511 39.624511) (width 0.25) (layer "B.Cu") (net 13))
 (segment (start 94 36.1) (end 97.524511 39.624511) (width 0.25) (layer "B.Cu") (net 13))
 (segment (start 133.894511 39.624511) (end 135 40.73) (width 0.25) (layer "B.Cu") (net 13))
 (segment (start 153.46 26.24) (end 153.51 26.29) (width 0.25) (layer "F.Cu") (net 12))
 (segment (start 143.2 26.24) (end 153.46 26.24) (width 0.25) (layer "F.Cu") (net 12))
 (segment (start 118 36.1) (end 132.91 36.1) (width 0.25) (layer "B.Cu") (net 12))
 (segment (start 132.91 36.1) (end 135 38.19) (width 0.25) (layer "B.Cu") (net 12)))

